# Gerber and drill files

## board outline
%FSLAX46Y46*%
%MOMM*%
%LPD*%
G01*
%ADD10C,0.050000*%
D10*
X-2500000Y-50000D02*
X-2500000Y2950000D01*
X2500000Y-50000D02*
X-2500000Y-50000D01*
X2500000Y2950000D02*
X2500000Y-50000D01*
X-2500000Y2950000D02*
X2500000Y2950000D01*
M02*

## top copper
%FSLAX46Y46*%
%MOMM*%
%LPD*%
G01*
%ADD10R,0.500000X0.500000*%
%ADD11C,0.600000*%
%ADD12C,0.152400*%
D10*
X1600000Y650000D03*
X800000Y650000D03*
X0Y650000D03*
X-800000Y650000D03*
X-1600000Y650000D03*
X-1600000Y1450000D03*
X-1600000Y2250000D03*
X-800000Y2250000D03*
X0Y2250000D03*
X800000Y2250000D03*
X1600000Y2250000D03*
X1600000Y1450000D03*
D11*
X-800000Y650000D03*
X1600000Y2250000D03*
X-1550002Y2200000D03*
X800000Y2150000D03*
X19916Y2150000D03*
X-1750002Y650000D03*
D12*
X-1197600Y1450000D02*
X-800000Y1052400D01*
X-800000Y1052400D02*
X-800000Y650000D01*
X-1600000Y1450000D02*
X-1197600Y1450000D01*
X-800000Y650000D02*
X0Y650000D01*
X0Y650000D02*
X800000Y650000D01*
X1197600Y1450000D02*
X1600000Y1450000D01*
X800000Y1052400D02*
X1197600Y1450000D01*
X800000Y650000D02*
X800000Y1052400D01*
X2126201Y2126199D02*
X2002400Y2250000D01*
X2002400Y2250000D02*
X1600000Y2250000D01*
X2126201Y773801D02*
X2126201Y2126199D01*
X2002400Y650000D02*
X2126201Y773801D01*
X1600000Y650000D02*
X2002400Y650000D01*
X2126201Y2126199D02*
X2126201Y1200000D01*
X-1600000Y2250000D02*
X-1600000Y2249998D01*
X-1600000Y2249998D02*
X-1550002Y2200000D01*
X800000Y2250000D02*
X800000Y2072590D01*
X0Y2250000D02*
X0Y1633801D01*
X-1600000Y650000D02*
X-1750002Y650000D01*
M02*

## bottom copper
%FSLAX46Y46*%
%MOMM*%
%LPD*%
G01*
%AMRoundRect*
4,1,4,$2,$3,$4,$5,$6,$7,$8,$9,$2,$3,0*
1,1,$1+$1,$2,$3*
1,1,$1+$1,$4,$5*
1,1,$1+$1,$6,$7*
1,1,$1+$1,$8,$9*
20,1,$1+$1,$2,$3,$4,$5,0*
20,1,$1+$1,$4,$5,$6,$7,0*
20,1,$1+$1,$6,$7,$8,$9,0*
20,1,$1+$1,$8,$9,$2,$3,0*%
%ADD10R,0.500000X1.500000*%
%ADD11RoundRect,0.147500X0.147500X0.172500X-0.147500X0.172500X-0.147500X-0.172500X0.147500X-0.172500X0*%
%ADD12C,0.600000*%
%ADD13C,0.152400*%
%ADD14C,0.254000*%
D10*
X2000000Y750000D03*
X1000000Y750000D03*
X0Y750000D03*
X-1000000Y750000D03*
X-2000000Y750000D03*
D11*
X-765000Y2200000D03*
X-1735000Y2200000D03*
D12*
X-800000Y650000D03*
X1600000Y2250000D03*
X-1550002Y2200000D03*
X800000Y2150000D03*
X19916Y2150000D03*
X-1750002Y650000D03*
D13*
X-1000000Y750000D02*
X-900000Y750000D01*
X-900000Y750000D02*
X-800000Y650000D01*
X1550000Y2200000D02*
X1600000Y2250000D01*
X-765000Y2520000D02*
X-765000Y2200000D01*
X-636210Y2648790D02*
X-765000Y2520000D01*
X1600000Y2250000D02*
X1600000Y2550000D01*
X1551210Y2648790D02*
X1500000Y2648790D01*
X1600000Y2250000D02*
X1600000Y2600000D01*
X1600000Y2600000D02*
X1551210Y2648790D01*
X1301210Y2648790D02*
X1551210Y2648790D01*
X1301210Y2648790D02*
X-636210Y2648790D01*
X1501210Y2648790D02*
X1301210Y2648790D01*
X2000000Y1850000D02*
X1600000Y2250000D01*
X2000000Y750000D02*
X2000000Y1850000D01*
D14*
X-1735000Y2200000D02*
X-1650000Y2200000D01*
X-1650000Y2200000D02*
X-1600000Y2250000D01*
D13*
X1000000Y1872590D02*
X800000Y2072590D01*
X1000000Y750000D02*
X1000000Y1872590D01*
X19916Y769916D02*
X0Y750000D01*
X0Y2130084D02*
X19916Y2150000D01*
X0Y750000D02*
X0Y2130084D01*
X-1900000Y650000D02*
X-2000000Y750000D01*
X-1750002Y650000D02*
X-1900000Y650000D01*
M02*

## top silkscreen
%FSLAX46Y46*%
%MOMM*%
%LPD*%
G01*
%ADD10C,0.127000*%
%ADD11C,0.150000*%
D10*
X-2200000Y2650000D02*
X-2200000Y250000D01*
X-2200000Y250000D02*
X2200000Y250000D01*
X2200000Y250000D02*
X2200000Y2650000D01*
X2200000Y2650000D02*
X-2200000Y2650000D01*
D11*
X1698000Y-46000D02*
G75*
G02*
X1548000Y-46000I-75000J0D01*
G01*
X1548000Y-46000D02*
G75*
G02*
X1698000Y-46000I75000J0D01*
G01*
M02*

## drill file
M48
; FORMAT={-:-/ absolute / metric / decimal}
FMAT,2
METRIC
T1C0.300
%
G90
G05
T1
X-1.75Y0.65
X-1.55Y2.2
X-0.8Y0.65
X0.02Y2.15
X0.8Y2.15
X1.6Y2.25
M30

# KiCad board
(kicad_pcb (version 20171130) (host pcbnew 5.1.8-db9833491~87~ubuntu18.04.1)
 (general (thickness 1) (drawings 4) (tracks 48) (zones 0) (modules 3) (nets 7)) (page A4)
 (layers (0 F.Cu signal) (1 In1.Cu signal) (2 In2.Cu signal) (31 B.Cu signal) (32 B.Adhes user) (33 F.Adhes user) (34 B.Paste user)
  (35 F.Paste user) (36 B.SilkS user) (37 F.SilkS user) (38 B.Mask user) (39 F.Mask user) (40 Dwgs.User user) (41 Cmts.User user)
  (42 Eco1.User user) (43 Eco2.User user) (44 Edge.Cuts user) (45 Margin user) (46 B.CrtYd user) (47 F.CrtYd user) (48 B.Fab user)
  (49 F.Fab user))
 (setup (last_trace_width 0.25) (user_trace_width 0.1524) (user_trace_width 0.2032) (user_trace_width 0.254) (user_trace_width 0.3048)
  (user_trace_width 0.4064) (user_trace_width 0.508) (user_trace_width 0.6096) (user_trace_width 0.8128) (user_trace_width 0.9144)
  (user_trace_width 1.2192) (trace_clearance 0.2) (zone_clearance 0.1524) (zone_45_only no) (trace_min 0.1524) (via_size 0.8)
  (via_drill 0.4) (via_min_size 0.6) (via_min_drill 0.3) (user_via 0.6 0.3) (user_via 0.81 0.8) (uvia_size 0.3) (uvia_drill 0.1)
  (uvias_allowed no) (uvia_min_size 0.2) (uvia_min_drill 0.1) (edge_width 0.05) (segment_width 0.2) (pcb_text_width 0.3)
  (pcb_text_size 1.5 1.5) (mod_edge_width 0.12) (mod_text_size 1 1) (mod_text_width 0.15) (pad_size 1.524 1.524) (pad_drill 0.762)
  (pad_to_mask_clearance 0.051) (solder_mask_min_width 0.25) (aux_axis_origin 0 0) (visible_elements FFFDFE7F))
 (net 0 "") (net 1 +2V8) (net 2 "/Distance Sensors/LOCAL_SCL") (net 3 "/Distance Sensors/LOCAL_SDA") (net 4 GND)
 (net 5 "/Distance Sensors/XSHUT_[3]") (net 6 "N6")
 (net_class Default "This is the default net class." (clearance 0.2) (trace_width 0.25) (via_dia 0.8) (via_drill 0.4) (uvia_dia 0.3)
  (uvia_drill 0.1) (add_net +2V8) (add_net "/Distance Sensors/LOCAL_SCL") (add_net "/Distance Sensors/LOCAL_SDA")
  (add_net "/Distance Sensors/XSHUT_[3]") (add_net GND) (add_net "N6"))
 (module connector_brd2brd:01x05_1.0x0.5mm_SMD (layer B.Cu) (at 0 -1.75)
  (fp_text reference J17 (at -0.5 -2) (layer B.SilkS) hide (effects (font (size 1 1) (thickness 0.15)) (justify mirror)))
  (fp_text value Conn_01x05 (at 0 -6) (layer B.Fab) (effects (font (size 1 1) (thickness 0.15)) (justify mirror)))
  (pad 5 smd rect (at 2 1 270) (size 1.5 0.5) (layers B.Cu B.Paste B.Mask) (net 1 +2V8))
  (pad 4 smd rect (at 1 1 270) (size 1.5 0.5) (layers B.Cu B.Paste B.Mask) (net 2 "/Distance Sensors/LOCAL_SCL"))
  (pad 3 smd rect (at 0 1 270) (size 1.5 0.5) (layers B.Cu B.Paste B.Mask) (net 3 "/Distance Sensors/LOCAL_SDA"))
  (pad 2 smd rect (at -1 1 270) (size 1.5 0.5) (layers B.Cu B.Paste B.Mask) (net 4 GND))
  (pad 1 smd rect (at -2 1 270) (size 1.5 0.5) (layers B.Cu B.Paste B.Mask) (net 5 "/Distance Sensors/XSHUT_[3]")))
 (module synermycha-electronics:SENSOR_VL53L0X (layer F.Cu) (at 0 -1.45 180)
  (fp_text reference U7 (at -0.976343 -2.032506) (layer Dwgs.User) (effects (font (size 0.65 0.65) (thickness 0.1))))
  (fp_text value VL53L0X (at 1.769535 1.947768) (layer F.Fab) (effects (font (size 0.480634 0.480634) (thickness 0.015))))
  (fp_line (start 2.2 1.2) (end 2.2 -1.2) (layer F.SilkS) (width 0.127))
  (fp_line (start 2.2 -1.2) (end -2.2 -1.2) (layer F.SilkS) (width 0.127))
  (fp_line (start -2.2 -1.2) (end -2.2 1.2) (layer F.SilkS) (width 0.127))
  (fp_line (start -2.2 1.2) (end 2.2 1.2) (layer F.SilkS) (width 0.127))
  (fp_circle (center -1.623 -1.496) (end -1.548 -1.496) (layer F.SilkS) (width 0.15))
  (pad 1 smd rect (at -1.6 -0.8 180) (size 0.5 0.5) (layers F.Cu F.Paste F.Mask) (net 1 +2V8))
  (pad 2 smd rect (at -0.8 -0.8 180) (size 0.5 0.5) (layers F.Cu F.Paste F.Mask) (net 4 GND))
  (pad 3 smd rect (at 0 -0.8 180) (size 0.5 0.5) (layers F.Cu F.Paste F.Mask) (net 4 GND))
  (pad 4 smd rect (at 0.8 -0.8 180) (size 0.5 0.5) (layers F.Cu F.Paste F.Mask) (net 4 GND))
  (pad 5 smd rect (at 1.6 -0.8 180) (size 0.5 0.5) (layers F.Cu F.Paste F.Mask) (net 5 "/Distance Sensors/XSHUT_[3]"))
  (pad 6 smd rect (at 1.6 0 180) (size 0.5 0.5) (layers F.Cu F.Paste F.Mask) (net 4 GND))
  (pad 7 smd rect (at 1.6 0.8 180) (size 0.5 0.5) (layers F.Cu F.Paste F.Mask) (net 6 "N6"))
  (pad 8 smd rect (at 0.8 0.8 180) (size 0.5 0.5) (layers F.Cu F.Paste F.Mask))
  (pad 9 smd rect (at 0 0.8 180) (size 0.5 0.5) (layers F.Cu F.Paste F.Mask) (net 3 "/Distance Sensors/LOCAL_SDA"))
  (pad 10 smd rect (at -0.8 0.8 180) (size 0.5 0.5) (layers F.Cu F.Paste F.Mask) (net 2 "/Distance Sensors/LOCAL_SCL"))
  (pad 11 smd rect (at -1.6 0.8 180) (size 0.5 0.5) (layers F.Cu F.Paste F.Mask) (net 1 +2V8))
  (pad 12 smd rect (at -1.6 0 180) (size 0.5 0.5) (layers F.Cu F.Paste F.Mask) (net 4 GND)))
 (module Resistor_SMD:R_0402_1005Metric (layer B.Cu) (at -1.25 -2.2 180)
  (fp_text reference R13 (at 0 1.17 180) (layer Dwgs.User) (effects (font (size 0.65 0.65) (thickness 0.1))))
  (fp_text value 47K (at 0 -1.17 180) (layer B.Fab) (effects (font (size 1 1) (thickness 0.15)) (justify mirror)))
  (pad 1 smd roundrect (at -0.485 0 180) (size 0.59 0.64) (layers B.Cu B.Paste B.Mask) (roundrect_rratio 0.25) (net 1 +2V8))
  (pad 2 smd roundrect (at 0.485 0 180) (size 0.59 0.64) (layers B.Cu B.Paste B.Mask) (roundrect_rratio 0.25) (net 6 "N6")))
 (gr_line (start -2.5 0.05) (end -2.5 -2.95) (layer Edge.Cuts) (width 0.05))
 (gr_line (start 2.5 0.05) (end -2.5 0.05) (layer Edge.Cuts) (width 0.05))
 (gr_line (start 2.5 -2.95) (end 2.5 0.05) (layer Edge.Cuts) (width 0.05))
 (gr_line (start -2.5 -2.95) (end 2.5 -2.95) (layer Edge.Cuts) (width 0.05))
 (segment (start -1.1976 -1.45) (end -0.8 -1.0524) (width 0.1524) (layer F.Cu) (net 4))
 (segment (start -0.8 -1.0524) (end -0.8 -0.65) (width 0.1524) (layer F.Cu) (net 4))
 (segment (start -1.6 -1.45) (end -1.1976 -1.45) (width 0.1524) (layer F.Cu) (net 4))
 (segment (start -0.8 -0.65) (end 0 -0.65) (width 0.1524) (layer F.Cu) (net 4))
 (segment (start 0 -0.65) (end 0.8 -0.65) (width 0.1524) (layer F.Cu) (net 4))
 (segment (start 1.1976 -1.45) (end 1.6 -1.45) (width 0.1524) (layer F.Cu) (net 4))
 (segment (start 0.8 -1.0524) (end 1.1976 -1.45) (width 0.1524) (layer F.Cu) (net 4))
 (segment (start 0.8 -0.65) (end 0.8 -1.0524) (width 0.1524) (layer F.Cu) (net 4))
 (via (at -0.8 -0.65) (size 0.6) (drill 0.3) (layers F.Cu B.Cu) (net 4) (status 1000000))
 (segment (start -1 -0.75) (end -0.9 -0.75) (width 0.1524) (layer B.Cu) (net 4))
 (segment (start -0.9 -0.75) (end -0.8 -0.65) (width 0.1524) (layer B.Cu) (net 4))
 (segment (start 2.126201 -2.126199) (end 2.0024 -2.25) (width 0.1524) (layer F.Cu) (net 1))
 (segment (start 2.0024 -2.25) (end 1.6 -2.25) (width 0.1524) (layer F.Cu) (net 1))
 (segment (start 2.126201 -0.773801) (end 2.126201 -2.126199) (width 0.1524) (layer F.Cu) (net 1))
 (segment (start 2.0024 -0.65) (end 2.126201 -0.773801) (width 0.1524) (layer F.Cu) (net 1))
 (segment (start 1.6 -0.65) (end 2.0024 -0.65) (width 0.1524) (layer F.Cu) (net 1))
 (via (at 1.6 -2.25) (size 0.6) (drill 0.3) (layers F.Cu B.Cu) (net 1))
 (segment (start 1.55 -2.2) (end 1.6 -2.25) (width 0.1524) (layer B.Cu) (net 1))
 (segment (start -0.765 -2.52) (end -0.765 -2.2) (width 0.1524) (layer B.Cu) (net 1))
 (segment (start -0.63621 -2.64879) (end -0.765 -2.52) (width 0.1524) (layer B.Cu) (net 1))
 (segment (start 1.6 -2.25) (end 1.6 -2.55) (width 0.1524) (layer B.Cu) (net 1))
 (segment (start 2.126201 -2.126199) (end 2.126201 -1.2) (width 0.1524) (layer F.Cu) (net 1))
 (segment (start 1.55121 -2.64879) (end 1.5 -2.64879) (width 0.1524) (layer B.Cu) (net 1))
 (segment (start 1.6 -2.25) (end 1.6 -2.6) (width 0.1524) (layer B.Cu) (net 1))
 (segment (start 1.6 -2.6) (end 1.55121 -2.64879) (width 0.1524) (layer B.Cu) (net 1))
 (segment (start 1.30121 -2.64879) (end 1.55121 -2.64879) (width 0.1524) (layer B.Cu) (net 1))
 (segment (start 1.30121 -2.64879) (end -0.63621 -2.64879) (width 0.1524) (layer B.Cu) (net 1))
 (segment (start 1.50121 -2.64879) (end 1.30121 -2.64879) (width 0.1524) (layer B.Cu) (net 1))
 (segment (start 2 -1.85) (end 1.6 -2.25) (width 0.1524) (layer B.Cu) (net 1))
 (segment (start 2 -0.75) (end 2 -1.85) (width 0.1524) (layer B.Cu) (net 1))
 (segment (start -1.735 -2.2) (end -1.65 -2.2) (width 0.254) (layer B.Cu) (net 6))
 (segment (start -1.65 -2.2) (end -1.6 -2.25) (width 0.254) (layer B.Cu) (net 6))
 (via (at -1.550002 -2.2) (size 0.6) (drill 0.3) (layers F.Cu B.Cu) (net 6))
 (segment (start -1.6 -2.25) (end -1.6 -2.249998) (width 0.1524) (layer F.Cu) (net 6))
 (segment (start -1.6 -2.249998) (end -1.550002 -2.2) (width 0.1524) (layer F.Cu) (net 6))
 (via (at 0.8 -2.15) (size 0.6) (drill 0.3) (layers F.Cu B.Cu) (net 2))
 (segment (start 0.8 -2.25) (end 0.8 -2.07259) (width 0.1524) (layer F.Cu) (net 2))
 (segment (start 1 -1.87259) (end 0.8 -2.07259) (width 0.1524) (layer B.Cu) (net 2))
 (segment (start 1 -0.75) (end 1 -1.87259) (width 0.1524) (layer B.Cu) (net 2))
 (via (at 0.019916 -2.15) (size 0.6) (drill 0.3) (layers F.Cu B.Cu) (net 3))
 (segment (start 0 -2.25) (end 0 -1.633801) (width 0.1524) (layer F.Cu) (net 3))
 (segment (start 0.019916 -0.769916) (end 0 -0.75) (width 0.1524) (layer B.Cu) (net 3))
 (segment (start 0 -2.130084) (end 0.019916 -2.15) (width 0.1524) (layer B.Cu) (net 3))
 (segment (start 0 -0.75) (end 0 -2.130084) (width 0.1524) (layer B.Cu) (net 3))
 (via (at -1.750002 -0.65) (size 0.6) (drill 0.3) (layers F.Cu B.Cu) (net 5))
 (segment (start -1.6 -0.65) (end -1.750002 -0.65) (width 0.1524) (layer F.Cu) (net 5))
 (segment (start -1.9 -0.65) (end -2 -0.75) (width 0.1524) (layer B.Cu) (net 5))
 (segment (start -1.750002 -0.65) (end -1.9 -0.65) (width 0.1524) (layer B.Cu) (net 5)))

